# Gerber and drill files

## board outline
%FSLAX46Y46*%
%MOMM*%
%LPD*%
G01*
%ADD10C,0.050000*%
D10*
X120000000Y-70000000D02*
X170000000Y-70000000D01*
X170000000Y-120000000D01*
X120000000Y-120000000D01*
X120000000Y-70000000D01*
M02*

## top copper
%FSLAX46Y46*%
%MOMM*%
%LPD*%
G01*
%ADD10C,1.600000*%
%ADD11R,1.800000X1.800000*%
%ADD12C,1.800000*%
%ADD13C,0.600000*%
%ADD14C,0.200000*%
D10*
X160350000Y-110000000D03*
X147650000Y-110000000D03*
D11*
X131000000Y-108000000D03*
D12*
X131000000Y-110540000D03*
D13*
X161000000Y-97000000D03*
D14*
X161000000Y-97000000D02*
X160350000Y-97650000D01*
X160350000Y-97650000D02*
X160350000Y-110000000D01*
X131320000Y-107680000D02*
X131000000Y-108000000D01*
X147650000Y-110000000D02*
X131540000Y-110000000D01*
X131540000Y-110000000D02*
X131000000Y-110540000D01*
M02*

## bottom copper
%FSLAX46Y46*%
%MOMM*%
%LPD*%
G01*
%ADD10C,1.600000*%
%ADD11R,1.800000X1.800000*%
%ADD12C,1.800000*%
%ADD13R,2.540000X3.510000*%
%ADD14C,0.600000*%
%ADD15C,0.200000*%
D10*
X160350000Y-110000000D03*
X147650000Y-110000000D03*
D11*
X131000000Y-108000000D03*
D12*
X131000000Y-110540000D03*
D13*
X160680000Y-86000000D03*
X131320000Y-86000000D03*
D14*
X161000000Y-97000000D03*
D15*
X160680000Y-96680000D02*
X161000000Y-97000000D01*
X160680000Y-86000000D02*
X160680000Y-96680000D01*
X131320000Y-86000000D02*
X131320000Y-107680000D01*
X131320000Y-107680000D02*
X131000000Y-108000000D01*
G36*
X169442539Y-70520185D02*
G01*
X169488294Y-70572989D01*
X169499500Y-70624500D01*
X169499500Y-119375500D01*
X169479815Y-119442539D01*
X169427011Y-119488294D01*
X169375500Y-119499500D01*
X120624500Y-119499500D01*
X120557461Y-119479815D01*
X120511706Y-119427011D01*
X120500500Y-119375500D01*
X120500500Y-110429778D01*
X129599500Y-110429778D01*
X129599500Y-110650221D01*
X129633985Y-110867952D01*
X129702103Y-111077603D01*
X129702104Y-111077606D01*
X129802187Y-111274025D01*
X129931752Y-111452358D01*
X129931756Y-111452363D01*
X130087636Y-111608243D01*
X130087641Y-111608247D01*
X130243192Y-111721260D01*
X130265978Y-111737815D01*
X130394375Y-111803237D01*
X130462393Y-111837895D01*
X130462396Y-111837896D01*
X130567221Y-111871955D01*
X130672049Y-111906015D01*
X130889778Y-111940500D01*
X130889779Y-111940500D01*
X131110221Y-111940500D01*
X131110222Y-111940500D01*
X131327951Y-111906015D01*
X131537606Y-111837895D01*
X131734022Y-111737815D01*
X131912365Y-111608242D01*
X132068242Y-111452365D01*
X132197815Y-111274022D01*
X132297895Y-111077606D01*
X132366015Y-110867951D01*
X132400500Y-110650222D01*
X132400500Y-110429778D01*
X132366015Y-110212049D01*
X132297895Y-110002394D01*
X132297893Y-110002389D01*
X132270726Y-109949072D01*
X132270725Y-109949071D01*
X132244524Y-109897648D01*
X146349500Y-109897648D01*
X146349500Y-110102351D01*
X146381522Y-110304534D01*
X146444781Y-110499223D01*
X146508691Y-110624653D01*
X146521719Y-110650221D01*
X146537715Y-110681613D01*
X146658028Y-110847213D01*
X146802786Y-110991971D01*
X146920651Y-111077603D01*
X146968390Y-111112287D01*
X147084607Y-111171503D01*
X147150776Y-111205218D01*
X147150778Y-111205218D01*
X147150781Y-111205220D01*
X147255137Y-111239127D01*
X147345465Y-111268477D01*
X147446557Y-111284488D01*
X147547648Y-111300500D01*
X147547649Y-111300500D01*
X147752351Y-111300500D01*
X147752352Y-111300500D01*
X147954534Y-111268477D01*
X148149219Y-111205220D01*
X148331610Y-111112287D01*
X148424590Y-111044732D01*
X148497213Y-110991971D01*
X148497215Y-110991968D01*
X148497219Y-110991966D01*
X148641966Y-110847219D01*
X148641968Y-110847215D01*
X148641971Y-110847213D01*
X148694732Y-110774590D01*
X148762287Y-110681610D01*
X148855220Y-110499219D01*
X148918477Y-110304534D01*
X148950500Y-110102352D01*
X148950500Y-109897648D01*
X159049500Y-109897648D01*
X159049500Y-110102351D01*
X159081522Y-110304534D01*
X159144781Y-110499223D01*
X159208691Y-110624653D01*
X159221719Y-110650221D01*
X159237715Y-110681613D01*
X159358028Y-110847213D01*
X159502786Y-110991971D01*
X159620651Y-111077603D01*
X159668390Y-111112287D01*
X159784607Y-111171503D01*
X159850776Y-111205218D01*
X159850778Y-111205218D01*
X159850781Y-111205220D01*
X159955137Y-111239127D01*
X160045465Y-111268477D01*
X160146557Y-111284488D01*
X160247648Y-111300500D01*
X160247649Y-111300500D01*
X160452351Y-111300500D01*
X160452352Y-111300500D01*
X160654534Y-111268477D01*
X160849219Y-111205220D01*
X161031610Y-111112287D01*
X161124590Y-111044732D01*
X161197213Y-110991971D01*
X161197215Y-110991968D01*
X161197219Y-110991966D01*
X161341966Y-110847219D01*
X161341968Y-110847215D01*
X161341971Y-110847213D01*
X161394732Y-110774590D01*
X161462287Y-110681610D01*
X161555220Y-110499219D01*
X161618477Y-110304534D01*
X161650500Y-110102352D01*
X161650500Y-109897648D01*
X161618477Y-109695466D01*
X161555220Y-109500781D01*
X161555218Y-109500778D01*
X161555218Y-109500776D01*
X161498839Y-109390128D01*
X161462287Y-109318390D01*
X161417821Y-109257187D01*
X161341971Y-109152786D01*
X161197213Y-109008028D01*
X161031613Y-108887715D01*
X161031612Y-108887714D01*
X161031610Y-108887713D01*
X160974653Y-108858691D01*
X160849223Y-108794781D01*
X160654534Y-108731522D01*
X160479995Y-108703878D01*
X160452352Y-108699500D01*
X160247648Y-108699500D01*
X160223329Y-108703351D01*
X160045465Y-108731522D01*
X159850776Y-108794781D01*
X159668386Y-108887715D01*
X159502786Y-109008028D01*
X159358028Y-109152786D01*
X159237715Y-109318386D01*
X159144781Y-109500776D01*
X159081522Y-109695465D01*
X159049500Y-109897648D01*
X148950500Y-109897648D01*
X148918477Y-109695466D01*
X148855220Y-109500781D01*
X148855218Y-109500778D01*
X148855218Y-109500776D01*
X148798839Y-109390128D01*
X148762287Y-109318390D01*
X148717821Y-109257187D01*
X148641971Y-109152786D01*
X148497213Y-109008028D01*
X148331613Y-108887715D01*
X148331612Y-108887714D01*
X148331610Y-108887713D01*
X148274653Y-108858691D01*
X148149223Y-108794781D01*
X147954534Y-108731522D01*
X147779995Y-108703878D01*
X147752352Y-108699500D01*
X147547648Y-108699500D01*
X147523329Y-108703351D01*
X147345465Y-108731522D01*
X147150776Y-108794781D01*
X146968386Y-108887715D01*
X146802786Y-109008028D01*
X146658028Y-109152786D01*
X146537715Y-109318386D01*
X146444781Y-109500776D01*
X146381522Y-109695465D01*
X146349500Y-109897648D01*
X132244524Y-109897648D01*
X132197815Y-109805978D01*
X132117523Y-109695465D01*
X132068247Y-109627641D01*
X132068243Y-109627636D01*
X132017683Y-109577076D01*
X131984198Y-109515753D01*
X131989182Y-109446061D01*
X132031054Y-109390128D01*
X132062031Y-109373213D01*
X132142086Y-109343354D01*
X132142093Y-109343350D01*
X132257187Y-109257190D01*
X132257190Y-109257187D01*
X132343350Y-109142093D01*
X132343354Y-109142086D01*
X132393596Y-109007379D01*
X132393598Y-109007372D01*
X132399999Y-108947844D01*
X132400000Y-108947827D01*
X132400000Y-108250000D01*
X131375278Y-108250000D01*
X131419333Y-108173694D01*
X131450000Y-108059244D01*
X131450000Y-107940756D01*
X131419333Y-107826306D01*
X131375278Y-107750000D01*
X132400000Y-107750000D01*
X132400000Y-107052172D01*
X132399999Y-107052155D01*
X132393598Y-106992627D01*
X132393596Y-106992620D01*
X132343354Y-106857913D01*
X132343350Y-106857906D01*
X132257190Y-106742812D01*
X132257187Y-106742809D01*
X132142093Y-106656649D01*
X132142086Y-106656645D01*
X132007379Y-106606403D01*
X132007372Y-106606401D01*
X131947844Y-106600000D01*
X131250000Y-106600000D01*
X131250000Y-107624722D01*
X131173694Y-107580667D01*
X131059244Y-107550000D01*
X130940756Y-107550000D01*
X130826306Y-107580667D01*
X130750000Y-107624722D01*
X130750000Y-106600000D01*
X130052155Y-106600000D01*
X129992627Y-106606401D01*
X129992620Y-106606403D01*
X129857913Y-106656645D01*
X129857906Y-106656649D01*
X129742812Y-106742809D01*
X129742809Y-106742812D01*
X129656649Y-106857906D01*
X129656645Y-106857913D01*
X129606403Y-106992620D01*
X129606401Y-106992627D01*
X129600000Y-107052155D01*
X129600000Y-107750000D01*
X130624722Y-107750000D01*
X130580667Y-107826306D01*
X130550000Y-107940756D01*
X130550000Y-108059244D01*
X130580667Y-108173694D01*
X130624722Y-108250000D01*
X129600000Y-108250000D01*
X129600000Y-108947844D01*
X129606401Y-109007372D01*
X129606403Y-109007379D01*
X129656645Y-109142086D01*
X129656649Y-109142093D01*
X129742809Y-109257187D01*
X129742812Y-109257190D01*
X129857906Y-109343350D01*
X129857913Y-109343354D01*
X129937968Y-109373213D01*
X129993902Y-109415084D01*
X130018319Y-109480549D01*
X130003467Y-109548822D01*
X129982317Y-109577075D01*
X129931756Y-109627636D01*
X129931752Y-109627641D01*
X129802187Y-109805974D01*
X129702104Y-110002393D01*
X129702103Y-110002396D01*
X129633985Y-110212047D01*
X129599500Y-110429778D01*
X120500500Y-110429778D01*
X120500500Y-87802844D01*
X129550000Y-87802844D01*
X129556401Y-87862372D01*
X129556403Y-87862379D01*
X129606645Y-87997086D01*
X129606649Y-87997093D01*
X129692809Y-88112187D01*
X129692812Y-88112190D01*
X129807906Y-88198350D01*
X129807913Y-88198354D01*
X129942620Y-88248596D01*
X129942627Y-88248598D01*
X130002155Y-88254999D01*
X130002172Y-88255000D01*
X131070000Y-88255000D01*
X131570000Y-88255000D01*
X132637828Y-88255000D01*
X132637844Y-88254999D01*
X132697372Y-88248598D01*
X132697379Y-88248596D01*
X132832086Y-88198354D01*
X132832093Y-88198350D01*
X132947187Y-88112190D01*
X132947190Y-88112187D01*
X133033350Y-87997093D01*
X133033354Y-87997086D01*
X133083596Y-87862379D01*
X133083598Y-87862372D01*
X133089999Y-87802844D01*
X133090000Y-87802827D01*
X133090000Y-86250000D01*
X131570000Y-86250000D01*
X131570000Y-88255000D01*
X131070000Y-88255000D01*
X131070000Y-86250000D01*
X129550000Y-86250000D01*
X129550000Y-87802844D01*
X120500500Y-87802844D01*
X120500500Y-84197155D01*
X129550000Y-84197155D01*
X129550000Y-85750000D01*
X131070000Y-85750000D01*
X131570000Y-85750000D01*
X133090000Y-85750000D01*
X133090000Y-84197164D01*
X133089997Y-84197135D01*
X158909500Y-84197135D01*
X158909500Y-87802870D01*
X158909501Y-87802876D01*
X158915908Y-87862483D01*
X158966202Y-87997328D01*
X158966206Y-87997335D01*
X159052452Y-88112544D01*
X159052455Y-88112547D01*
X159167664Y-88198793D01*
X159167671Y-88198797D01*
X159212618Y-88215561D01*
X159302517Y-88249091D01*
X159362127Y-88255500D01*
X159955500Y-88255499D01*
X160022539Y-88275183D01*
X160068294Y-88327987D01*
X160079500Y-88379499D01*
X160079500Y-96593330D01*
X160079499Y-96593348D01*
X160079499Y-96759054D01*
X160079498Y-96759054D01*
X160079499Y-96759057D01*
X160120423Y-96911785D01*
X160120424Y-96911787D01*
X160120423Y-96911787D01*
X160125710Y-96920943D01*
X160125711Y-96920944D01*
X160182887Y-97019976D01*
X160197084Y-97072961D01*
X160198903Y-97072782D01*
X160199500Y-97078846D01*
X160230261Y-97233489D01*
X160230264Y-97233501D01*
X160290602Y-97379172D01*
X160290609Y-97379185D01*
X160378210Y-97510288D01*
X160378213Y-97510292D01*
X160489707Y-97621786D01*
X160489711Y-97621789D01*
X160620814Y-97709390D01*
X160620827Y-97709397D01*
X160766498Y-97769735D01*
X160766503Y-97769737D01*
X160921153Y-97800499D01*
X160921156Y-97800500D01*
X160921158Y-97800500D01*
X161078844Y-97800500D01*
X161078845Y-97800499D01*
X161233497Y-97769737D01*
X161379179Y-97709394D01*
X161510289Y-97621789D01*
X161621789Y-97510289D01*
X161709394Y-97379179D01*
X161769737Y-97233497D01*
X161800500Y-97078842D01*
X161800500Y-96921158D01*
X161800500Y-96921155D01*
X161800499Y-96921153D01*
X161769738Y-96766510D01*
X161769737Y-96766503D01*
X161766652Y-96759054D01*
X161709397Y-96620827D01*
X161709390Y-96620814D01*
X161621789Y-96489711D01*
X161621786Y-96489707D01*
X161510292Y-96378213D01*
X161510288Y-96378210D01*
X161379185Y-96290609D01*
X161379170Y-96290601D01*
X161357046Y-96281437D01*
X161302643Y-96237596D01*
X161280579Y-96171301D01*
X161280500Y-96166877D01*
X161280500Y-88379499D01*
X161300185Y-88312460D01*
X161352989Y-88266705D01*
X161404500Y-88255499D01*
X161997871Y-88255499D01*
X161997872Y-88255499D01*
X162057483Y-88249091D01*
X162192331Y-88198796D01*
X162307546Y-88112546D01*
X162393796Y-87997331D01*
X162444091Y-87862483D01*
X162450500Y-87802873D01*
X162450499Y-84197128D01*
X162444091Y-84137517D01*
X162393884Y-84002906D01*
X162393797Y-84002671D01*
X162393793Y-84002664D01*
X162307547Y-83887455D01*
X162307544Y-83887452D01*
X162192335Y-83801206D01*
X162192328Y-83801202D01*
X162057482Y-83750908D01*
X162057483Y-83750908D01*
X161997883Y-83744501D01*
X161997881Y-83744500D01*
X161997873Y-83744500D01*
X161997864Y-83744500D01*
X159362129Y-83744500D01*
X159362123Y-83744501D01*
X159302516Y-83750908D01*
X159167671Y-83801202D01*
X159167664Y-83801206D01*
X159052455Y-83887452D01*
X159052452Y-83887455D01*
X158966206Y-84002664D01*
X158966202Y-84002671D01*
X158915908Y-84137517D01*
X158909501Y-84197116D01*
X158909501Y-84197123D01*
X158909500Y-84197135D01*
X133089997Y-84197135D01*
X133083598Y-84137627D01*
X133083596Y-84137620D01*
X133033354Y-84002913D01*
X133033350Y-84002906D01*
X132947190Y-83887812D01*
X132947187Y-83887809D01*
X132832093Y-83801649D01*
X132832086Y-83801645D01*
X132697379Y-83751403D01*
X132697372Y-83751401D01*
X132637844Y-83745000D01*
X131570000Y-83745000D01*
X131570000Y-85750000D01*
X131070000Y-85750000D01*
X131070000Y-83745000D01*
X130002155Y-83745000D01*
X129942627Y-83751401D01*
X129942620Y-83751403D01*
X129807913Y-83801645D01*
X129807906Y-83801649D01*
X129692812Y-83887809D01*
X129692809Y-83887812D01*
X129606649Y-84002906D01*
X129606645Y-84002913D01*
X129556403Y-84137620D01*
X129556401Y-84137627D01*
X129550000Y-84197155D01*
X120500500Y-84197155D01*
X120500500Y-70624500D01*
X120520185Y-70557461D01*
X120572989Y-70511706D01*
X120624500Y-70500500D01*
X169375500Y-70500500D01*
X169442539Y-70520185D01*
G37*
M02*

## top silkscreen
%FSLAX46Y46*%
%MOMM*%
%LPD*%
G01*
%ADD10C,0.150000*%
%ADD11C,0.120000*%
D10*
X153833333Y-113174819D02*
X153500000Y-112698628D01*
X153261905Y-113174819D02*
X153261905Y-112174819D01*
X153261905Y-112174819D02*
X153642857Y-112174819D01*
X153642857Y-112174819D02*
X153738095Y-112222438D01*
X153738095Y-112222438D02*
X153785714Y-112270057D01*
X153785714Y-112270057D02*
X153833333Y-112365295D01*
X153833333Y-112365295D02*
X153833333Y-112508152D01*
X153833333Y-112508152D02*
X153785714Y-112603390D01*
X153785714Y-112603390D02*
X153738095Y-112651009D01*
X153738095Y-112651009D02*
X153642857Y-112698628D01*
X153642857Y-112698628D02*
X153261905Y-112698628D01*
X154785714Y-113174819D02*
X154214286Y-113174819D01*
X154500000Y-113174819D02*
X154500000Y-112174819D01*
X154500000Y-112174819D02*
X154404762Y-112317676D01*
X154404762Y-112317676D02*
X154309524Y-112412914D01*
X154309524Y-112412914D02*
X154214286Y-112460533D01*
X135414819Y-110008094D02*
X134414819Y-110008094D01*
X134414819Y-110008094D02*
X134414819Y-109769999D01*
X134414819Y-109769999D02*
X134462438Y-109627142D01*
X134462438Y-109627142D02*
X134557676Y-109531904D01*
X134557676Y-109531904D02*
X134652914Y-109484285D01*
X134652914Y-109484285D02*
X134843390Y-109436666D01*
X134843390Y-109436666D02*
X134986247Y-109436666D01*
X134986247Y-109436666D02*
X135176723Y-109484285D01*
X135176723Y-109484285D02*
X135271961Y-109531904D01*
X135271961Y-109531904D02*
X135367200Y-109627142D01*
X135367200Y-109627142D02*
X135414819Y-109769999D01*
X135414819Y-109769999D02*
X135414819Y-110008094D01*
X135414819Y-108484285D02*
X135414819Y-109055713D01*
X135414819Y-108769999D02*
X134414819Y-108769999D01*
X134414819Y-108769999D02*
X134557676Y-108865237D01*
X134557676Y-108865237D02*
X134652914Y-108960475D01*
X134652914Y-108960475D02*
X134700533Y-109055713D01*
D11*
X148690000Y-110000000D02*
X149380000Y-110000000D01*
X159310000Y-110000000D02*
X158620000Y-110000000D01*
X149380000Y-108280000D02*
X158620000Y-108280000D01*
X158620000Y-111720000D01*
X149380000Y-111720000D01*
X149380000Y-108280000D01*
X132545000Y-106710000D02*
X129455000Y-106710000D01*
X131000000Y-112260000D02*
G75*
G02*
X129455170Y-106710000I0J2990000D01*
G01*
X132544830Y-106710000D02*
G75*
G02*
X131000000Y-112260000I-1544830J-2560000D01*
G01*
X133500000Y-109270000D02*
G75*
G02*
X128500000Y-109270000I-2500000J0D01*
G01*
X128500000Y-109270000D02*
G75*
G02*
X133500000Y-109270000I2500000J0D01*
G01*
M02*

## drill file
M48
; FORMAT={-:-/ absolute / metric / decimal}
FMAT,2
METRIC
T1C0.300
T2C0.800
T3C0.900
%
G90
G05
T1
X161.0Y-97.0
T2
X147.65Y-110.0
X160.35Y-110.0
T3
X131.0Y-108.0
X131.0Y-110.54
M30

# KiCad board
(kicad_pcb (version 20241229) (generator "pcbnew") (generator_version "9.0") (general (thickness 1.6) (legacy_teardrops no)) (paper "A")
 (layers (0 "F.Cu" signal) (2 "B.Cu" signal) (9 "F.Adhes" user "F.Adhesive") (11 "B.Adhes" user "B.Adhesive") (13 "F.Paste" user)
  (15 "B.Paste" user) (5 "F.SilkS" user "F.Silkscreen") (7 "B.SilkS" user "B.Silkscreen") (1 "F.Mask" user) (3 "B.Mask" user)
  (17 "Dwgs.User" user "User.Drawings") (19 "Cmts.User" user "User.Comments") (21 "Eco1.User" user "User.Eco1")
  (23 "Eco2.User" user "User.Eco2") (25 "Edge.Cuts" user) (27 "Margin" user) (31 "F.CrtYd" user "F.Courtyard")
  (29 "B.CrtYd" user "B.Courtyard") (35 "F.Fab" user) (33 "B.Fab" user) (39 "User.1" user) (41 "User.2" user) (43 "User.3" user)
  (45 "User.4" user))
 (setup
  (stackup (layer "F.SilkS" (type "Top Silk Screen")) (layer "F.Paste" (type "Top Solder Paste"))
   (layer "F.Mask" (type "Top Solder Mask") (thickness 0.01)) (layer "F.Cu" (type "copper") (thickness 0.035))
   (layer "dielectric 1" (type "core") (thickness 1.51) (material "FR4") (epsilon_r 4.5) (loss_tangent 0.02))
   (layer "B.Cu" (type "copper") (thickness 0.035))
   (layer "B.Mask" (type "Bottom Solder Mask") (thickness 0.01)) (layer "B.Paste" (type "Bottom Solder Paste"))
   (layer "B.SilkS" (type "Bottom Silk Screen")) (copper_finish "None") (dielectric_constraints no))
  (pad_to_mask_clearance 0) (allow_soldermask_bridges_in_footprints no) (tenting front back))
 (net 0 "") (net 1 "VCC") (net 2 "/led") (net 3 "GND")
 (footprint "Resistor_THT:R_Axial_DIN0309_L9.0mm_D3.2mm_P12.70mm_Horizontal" (layer "F.Cu") (at 160.35 110 180)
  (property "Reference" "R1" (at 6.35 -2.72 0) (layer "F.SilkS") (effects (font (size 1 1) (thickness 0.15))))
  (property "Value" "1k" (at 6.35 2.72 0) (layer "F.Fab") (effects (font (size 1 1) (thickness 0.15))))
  (fp_line (start 11.66 0) (end 10.97 0) (stroke (width 0.12) (type solid)) (layer "F.SilkS"))
  (fp_line (start 1.04 0) (end 1.73 0) (stroke (width 0.12) (type solid)) (layer "F.SilkS"))
  (fp_rect (start 1.73 -1.72) (end 10.97 1.72) (stroke (width 0.12) (type solid)) (fill no) (layer "F.SilkS"))
  (pad "1" thru_hole circle (at 0 0 180) (size 1.6 1.6) (drill 0.8) (layers "*.Cu" "*.Mask") (remove_unused_layers no) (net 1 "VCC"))
  (pad "2" thru_hole circle (at 12.7 0 180) (size 1.6 1.6) (drill 0.8) (layers "*.Cu" "*.Mask") (remove_unused_layers no) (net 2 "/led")))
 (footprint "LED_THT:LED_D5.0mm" (layer "F.Cu") (at 131 108 -90)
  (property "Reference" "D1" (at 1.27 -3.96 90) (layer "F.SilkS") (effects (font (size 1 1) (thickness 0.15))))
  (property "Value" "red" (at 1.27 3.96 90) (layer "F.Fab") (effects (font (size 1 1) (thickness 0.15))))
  (fp_line (start -1.29 -1.545) (end -1.29 1.545) (stroke (width 0.12) (type solid)) (layer "F.SilkS"))
  (fp_arc (start 4.26 0) (mid 2.071779 2.880495) (end -1.29 1.54483) (stroke (width 0.12) (type solid)) (layer "F.SilkS"))
  (fp_arc (start -1.29 -1.54483) (mid 2.071779 -2.880495) (end 4.26 0) (stroke (width 0.12) (type solid)) (layer "F.SilkS"))
  (fp_circle (center 1.27 0) (end 3.77 0) (stroke (width 0.12) (type solid)) (fill no) (layer "F.SilkS"))
  (pad "1" thru_hole rect (at 0 0 270) (size 1.8 1.8) (drill 0.9) (layers "*.Cu" "*.Mask") (remove_unused_layers no) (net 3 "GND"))
  (pad "2" thru_hole circle (at 2.54 0 270) (size 1.8 1.8) (drill 0.9) (layers "*.Cu" "*.Mask") (remove_unused_layers no) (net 2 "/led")))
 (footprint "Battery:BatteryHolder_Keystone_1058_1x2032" (layer "B.Cu") (at 146 86 180)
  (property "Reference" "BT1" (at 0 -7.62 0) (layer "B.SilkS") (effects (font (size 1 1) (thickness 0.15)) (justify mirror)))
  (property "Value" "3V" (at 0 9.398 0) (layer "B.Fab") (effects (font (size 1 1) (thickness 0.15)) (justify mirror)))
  (pad "1" smd rect (at -14.68 0 180) (size 2.54 3.51) (layers "B.Cu" "B.Mask" "B.Paste") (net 1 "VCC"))
  (pad "2" smd rect (at 14.68 0 180) (size 2.54 3.51) (layers "B.Cu" "B.Mask" "B.Paste") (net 3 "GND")))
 (gr_rect (start 120 70) (end 170 120) (stroke (width 0.05) (type default)) (fill no) (layer "Edge.Cuts"))
 (segment (start 161 97) (end 160.35 97.65) (width 0.2) (layer "F.Cu") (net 1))
 (segment (start 160.35 97.65) (end 160.35 110) (width 0.2) (layer "F.Cu") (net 1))
 (via (at 161 97) (size 0.6) (drill 0.3) (layers "F.Cu" "B.Cu") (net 1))
 (segment (start 160.68 96.68) (end 161 97) (width 0.2) (layer "B.Cu") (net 1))
 (segment (start 160.68 86) (end 160.68 96.68) (width 0.2) (layer "B.Cu") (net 1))
 (segment (start 131.32 107.68) (end 131 108) (width 0.2) (layer "F.Cu") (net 3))
 (segment (start 131.32 86) (end 131.32 107.68) (width 0.2) (layer "B.Cu") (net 3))
 (segment (start 131.32 107.68) (end 131 108) (width 0.2) (layer "B.Cu") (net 3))
 (segment (start 147.65 110) (end 131.54 110) (width 0.2) (layer "F.Cu") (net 2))
 (segment (start 131.54 110) (end 131 110.54) (width 0.2) (layer "F.Cu") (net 2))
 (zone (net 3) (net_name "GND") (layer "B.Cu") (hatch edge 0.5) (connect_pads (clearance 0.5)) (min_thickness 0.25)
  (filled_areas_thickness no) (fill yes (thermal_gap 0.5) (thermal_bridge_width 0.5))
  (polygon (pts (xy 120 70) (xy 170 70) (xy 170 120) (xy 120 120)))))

